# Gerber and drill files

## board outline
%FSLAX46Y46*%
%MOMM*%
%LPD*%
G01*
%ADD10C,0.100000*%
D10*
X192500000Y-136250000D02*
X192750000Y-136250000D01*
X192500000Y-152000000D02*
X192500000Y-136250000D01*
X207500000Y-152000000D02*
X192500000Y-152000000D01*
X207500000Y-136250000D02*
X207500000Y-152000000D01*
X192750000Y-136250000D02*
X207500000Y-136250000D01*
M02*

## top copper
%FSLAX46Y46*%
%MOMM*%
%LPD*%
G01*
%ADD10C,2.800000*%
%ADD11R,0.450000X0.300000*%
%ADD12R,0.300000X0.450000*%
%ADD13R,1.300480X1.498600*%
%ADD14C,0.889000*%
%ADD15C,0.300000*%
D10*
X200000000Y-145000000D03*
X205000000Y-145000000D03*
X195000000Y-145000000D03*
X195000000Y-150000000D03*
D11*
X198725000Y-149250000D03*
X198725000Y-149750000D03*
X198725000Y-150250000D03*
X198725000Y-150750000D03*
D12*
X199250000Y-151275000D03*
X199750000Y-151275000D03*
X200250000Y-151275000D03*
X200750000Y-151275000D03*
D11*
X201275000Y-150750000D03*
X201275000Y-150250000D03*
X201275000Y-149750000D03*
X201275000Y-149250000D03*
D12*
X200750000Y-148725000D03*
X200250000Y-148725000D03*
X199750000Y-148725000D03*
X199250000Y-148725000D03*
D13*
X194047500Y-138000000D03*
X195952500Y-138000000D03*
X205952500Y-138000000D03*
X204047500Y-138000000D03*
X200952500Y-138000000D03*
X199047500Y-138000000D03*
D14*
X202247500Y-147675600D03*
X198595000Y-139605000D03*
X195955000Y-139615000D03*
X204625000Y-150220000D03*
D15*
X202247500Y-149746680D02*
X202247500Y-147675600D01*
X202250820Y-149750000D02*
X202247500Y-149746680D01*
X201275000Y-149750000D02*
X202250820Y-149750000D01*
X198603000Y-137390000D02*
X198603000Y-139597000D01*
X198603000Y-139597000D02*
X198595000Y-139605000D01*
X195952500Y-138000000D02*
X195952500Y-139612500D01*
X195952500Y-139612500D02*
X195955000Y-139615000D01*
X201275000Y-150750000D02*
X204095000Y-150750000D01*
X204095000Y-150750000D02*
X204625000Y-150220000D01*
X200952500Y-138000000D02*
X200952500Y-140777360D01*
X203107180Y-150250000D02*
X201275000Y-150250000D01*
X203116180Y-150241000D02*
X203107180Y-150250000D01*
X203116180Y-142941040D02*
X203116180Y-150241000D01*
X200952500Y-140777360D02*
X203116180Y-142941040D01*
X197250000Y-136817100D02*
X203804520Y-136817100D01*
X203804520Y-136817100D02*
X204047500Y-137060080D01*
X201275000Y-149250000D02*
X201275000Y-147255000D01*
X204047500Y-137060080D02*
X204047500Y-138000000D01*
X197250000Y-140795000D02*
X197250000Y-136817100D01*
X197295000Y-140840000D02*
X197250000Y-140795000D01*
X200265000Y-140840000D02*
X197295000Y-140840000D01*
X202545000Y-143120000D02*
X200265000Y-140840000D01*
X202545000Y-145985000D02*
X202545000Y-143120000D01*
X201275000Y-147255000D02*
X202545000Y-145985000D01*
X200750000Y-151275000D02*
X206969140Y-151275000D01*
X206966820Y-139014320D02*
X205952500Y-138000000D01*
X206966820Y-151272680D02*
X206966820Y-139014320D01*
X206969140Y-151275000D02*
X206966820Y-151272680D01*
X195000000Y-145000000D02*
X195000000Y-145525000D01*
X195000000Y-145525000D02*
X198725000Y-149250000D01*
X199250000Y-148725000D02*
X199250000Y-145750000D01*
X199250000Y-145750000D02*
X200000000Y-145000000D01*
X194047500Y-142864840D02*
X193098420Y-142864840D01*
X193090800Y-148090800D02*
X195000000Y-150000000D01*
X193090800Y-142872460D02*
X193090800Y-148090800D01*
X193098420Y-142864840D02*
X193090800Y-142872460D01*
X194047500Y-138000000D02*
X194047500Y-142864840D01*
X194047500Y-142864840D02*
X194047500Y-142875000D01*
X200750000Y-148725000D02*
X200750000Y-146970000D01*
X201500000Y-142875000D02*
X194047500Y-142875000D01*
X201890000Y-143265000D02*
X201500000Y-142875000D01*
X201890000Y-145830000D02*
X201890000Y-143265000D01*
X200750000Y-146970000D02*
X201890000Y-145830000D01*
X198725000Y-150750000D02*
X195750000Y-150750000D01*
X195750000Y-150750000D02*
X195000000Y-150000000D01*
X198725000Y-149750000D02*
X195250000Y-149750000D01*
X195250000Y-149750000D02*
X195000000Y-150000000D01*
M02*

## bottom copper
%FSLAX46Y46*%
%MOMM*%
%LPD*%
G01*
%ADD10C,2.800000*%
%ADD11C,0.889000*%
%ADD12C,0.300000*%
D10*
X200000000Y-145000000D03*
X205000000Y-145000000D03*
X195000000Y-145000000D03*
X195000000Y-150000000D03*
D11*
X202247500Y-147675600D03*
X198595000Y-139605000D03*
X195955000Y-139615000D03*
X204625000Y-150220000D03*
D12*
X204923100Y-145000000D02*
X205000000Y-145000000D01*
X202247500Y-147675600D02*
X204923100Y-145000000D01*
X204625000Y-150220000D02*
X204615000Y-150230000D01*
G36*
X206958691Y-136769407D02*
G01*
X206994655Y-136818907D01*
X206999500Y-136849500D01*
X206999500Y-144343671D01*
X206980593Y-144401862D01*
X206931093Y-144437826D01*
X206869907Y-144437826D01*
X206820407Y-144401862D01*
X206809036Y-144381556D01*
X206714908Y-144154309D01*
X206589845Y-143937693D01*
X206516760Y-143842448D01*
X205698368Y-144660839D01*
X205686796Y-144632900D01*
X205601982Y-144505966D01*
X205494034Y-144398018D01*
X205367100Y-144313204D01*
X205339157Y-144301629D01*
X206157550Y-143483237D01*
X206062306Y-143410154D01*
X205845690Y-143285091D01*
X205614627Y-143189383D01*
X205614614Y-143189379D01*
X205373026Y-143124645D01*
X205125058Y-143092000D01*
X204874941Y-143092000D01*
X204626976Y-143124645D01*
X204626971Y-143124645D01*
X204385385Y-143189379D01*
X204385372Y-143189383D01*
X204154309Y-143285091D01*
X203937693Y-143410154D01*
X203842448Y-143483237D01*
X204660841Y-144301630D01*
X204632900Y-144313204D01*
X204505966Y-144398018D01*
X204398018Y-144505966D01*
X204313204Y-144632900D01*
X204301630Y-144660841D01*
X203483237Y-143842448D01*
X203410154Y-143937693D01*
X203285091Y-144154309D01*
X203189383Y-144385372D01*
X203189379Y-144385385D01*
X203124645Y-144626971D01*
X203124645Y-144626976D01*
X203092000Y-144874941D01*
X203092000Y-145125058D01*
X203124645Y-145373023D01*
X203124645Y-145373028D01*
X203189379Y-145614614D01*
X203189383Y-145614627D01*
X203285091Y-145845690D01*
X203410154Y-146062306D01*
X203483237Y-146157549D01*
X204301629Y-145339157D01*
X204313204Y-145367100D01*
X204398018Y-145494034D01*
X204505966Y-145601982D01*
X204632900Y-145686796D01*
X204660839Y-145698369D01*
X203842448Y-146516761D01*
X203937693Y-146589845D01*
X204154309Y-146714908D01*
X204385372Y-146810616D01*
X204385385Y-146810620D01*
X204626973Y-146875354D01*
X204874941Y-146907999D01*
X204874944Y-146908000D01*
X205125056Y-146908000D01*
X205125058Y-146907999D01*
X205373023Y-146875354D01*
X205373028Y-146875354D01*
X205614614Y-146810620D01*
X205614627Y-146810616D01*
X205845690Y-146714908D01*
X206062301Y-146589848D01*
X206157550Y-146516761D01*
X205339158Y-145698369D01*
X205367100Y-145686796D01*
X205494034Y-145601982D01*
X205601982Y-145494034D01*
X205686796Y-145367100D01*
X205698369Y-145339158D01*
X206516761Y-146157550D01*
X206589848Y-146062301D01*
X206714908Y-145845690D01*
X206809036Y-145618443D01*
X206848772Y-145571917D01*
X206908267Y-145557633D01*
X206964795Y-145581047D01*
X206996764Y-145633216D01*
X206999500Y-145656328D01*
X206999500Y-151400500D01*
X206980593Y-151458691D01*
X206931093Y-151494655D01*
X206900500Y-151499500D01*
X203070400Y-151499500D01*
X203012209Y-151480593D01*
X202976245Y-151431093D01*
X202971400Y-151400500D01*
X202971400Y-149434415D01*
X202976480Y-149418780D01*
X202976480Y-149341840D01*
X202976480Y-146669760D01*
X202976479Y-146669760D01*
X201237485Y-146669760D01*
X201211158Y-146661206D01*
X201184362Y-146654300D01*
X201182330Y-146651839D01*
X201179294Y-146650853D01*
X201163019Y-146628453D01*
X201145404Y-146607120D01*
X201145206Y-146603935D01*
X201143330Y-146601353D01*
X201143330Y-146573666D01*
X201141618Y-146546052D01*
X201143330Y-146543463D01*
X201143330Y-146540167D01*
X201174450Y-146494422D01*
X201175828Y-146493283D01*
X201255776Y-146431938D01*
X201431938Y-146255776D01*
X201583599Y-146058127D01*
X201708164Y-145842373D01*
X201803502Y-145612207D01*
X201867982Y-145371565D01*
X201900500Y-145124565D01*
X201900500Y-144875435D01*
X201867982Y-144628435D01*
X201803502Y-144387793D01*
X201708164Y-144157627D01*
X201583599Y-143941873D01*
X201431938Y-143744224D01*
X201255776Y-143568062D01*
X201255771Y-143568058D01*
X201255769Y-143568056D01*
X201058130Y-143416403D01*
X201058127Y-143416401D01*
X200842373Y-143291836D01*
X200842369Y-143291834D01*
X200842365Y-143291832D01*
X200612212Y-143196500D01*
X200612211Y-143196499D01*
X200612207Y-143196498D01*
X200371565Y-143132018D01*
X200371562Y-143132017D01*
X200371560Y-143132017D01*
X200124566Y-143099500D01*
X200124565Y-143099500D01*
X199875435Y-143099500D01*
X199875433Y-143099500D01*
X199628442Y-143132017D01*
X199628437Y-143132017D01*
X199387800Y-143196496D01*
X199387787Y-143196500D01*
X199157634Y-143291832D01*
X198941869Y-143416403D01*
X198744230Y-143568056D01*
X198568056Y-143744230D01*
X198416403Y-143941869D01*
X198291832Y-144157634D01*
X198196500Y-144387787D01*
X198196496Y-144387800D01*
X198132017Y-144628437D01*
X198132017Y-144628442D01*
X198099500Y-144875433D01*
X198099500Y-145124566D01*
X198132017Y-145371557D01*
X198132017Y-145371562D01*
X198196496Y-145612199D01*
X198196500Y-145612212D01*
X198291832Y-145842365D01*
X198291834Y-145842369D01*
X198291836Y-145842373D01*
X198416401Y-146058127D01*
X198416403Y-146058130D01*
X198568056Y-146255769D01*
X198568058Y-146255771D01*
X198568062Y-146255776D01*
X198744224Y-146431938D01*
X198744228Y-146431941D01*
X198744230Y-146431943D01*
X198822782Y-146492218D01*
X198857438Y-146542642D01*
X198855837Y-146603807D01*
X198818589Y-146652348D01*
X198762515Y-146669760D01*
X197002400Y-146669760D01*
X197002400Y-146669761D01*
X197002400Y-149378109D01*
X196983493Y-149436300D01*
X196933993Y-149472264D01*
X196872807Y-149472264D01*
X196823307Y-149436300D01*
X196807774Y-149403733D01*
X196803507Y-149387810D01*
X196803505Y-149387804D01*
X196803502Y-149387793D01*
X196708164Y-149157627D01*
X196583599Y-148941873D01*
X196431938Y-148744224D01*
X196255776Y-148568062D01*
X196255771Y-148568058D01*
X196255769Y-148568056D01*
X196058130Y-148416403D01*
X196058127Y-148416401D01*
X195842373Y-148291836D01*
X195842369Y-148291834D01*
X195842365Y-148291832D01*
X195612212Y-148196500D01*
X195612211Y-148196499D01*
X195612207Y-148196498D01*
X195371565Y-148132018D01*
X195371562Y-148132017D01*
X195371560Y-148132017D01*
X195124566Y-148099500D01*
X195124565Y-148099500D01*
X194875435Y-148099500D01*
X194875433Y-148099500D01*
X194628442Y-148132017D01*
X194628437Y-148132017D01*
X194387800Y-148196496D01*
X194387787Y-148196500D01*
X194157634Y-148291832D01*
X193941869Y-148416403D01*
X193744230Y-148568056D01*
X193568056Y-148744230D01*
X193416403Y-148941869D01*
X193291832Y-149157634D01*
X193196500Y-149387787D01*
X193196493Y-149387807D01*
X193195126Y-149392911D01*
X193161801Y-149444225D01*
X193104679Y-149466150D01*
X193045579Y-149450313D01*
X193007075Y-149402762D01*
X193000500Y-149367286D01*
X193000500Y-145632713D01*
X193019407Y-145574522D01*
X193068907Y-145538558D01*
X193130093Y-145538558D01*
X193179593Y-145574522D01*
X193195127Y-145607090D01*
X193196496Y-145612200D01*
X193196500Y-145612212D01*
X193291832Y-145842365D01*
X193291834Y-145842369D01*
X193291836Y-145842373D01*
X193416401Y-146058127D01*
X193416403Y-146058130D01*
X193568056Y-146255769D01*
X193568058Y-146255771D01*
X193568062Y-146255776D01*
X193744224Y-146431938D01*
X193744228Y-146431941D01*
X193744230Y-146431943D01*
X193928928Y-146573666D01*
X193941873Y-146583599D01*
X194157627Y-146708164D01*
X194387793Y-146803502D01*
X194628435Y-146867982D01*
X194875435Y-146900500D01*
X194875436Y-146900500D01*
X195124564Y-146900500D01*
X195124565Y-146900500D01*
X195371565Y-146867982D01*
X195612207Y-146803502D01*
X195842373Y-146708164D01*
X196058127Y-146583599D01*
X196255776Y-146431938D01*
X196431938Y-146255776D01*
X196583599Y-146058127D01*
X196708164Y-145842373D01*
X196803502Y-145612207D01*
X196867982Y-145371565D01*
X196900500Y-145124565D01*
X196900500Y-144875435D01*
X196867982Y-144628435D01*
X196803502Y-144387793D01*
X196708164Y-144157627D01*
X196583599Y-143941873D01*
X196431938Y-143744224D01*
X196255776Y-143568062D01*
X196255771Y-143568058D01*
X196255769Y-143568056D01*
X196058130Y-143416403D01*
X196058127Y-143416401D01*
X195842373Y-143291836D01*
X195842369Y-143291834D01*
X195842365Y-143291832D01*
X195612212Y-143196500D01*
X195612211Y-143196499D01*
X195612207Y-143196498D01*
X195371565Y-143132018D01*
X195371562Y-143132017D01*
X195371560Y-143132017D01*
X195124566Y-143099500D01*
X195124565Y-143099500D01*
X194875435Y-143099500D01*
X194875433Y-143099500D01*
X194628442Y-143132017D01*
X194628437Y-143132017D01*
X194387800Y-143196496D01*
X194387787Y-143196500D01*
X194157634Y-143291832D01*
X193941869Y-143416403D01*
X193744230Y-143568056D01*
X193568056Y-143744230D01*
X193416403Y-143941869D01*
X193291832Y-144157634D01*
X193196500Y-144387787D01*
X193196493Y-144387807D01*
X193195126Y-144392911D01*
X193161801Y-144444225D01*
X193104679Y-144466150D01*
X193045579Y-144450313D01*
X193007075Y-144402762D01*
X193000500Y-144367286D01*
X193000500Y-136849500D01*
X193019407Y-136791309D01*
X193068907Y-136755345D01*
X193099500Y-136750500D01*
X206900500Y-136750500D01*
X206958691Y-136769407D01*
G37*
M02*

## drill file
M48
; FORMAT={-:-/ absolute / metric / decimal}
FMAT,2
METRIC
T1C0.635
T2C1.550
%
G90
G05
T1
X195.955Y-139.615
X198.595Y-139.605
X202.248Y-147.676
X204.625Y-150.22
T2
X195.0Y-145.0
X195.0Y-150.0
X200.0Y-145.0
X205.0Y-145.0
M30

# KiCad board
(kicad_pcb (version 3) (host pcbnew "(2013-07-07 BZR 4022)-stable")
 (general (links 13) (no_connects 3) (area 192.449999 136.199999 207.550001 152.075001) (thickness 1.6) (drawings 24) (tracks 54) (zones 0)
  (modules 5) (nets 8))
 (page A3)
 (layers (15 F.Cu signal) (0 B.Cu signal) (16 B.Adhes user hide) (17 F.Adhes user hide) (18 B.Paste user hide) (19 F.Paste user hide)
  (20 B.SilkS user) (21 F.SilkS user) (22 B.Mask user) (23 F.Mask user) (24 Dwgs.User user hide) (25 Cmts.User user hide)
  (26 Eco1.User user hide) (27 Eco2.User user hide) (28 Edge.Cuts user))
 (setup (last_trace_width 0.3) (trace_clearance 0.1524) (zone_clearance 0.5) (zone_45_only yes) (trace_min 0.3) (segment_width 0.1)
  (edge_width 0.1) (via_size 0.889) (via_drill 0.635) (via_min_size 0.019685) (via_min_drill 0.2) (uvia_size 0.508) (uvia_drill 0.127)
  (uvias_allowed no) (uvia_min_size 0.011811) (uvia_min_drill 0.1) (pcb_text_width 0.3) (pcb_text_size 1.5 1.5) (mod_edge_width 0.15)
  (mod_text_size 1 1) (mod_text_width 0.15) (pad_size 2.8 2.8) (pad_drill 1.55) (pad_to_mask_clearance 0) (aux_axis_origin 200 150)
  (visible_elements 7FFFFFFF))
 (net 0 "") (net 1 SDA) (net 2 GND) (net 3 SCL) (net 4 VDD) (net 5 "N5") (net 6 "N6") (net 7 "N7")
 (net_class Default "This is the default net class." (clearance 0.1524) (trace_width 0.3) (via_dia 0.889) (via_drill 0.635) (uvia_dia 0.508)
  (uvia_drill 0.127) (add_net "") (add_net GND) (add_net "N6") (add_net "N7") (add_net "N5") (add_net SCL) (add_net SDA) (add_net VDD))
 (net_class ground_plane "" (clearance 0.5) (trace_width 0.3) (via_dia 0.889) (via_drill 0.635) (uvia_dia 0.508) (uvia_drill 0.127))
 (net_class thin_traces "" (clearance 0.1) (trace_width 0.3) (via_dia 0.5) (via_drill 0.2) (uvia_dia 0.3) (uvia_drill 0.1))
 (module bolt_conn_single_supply (layer F.Cu) (at 200 150)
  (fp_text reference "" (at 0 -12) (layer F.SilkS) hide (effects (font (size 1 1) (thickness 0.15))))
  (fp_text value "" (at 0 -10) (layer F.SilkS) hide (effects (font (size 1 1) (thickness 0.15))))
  (pad 4 thru_hole circle (at 0 -5) (size 2.8 2.8) (drill 1.55) (layers *.Cu F.SilkS F.Mask) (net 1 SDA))
  (pad 2 thru_hole circle (at 5 -5) (size 2.8 2.8) (drill 1.55) (layers *.Cu F.SilkS F.Mask) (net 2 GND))
  (pad 3 thru_hole circle (at -5 -5) (size 2.8 2.8) (drill 1.55) (layers *.Cu F.SilkS F.Mask) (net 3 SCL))
  (pad 1 thru_hole circle (at -5 0) (size 2.8 2.8) (drill 1.55) (layers *.Cu F.SilkS F.Mask) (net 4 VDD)))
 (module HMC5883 (layer F.Cu) (at 200 150)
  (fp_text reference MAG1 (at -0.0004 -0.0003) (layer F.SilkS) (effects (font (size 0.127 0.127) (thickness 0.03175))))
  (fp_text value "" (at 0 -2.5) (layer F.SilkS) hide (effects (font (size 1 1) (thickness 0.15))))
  (pad 1 smd rect (at -1.275 -0.75) (size 0.45 0.3) (layers F.Cu F.Paste F.Mask) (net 3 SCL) (clearance 0.05) (zone_connect 1))
  (pad 2 smd rect (at -1.275 -0.25) (size 0.45 0.3) (layers F.Cu F.Paste F.Mask) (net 4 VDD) (clearance 0.05))
  (pad 3 smd rect (at -1.275 0.25) (size 0.45 0.3) (layers F.Cu F.Paste F.Mask) (clearance 0.05))
  (pad 4 smd rect (at -1.275 0.75) (size 0.45 0.3) (layers F.Cu F.Paste F.Mask) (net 4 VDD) (clearance 0.05))
  (pad 5 smd rect (at -0.75 1.275 90) (size 0.45 0.3) (layers F.Cu F.Paste F.Mask) (clearance 0.05))
  (pad 6 smd rect (at -0.25 1.275 90) (size 0.45 0.3) (layers F.Cu F.Paste F.Mask) (clearance 0.05))
  (pad 7 smd rect (at 0.25 1.275 90) (size 0.45 0.3) (layers F.Cu F.Paste F.Mask) (clearance 0.05))
  (pad 8 smd rect (at 0.75 1.275 90) (size 0.45 0.3) (layers F.Cu F.Paste F.Mask) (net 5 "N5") (clearance 0.05))
  (pad 9 smd rect (at 1.275 0.75) (size 0.45 0.3) (layers F.Cu F.Paste F.Mask) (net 2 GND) (clearance 0.05))
  (pad 10 smd rect (at 1.275 0.25) (size 0.45 0.3) (layers F.Cu F.Paste F.Mask) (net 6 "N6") (clearance 0.05))
  (pad 11 smd rect (at 1.275 -0.25) (size 0.45 0.3) (layers F.Cu F.Paste F.Mask) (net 2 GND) (clearance 0.05))
  (pad 12 smd rect (at 1.275 -0.75) (size 0.45 0.3) (layers F.Cu F.Paste F.Mask) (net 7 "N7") (clearance 0.05))
  (pad 13 smd rect (at 0.75 -1.275 90) (size 0.45 0.3) (layers F.Cu F.Paste F.Mask) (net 4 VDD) (clearance 0.05))
  (pad 14 smd rect (at 0.25 -1.275 90) (size 0.45 0.3) (layers F.Cu F.Paste F.Mask) (clearance 0.05))
  (pad 15 smd rect (at -0.25 -1.275 90) (size 0.45 0.3) (layers F.Cu F.Paste F.Mask) (clearance 0.05))
  (pad 16 smd rect (at -0.75 -1.275 90) (size 0.45 0.3) (layers F.Cu F.Paste F.Mask) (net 1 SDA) (clearance 0.05)))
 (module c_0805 (layer F.Cu) (at 195 138 180)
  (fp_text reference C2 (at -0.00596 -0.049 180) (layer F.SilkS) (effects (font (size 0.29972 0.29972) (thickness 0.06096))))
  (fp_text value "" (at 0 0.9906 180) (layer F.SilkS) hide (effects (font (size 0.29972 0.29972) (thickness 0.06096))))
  (pad 1 smd rect (at 0.9525 0 180) (size 1.30048 1.4986) (layers F.Cu F.Paste F.Mask) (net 4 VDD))
  (pad 2 smd rect (at -0.9525 0 180) (size 1.30048 1.4986) (layers F.Cu F.Paste F.Mask) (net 2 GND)))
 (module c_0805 (layer F.Cu) (at 205 138)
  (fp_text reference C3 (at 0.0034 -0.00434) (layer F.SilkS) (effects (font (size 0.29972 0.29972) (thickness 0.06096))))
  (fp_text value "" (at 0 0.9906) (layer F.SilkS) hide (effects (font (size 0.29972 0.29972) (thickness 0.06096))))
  (pad 1 smd rect (at 0.9525 0) (size 1.30048 1.4986) (layers F.Cu F.Paste F.Mask) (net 5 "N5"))
  (pad 2 smd rect (at -0.9525 0) (size 1.30048 1.4986) (layers F.Cu F.Paste F.Mask) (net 7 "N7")))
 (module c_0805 (layer F.Cu) (at 200 138)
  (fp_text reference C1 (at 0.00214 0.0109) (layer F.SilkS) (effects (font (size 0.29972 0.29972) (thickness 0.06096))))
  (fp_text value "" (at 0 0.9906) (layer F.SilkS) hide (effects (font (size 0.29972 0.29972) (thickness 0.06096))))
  (pad 1 smd rect (at 0.9525 0) (size 1.30048 1.4986) (layers F.Cu F.Paste F.Mask) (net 6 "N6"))
  (pad 2 smd rect (at -0.9525 0) (size 1.30048 1.4986) (layers F.Cu F.Paste F.Mask) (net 2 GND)))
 (gr_line (start 192.5 136.25) (end 192.75 136.25) (angle 90) (layer Edge.Cuts) (width 0.1))
 (gr_line (start 192.5 152) (end 192.5 136.25) (angle 90) (layer Edge.Cuts) (width 0.1))
 (gr_line (start 207.5 152) (end 192.5 152) (angle 90) (layer Edge.Cuts) (width 0.1))
 (gr_line (start 207.5 136.25) (end 207.5 152) (angle 90) (layer Edge.Cuts) (width 0.1))
 (gr_line (start 192.75 136.25) (end 207.5 136.25) (angle 90) (layer Edge.Cuts) (width 0.1))
 (segment (start 204.9231 145) (end 205 145) (width 0.3) (layer B.Cu) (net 2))
 (segment (start 202.2475 147.6756) (end 204.9231 145) (width 0.3) (layer B.Cu) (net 2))
 (via (at 202.2475 147.6756) (size 0.889) (layers F.Cu B.Cu) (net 2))
 (segment (start 202.2475 149.74668) (end 202.2475 147.6756) (width 0.3) (layer F.Cu) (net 2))
 (segment (start 202.25082 149.75) (end 202.2475 149.74668) (width 0.3) (layer F.Cu) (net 2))
 (segment (start 201.275 149.75) (end 202.25082 149.75) (width 0.3) (layer F.Cu) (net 2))
 (segment (start 198.603 137.39) (end 198.603 139.597) (width 0.3) (layer F.Cu) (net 2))
 (via (at 198.595 139.605) (size 0.889) (layers F.Cu B.Cu) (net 2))
 (segment (start 198.603 139.597) (end 198.595 139.605) (width 0.3) (layer F.Cu) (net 2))
 (segment (start 195.9525 138) (end 195.9525 139.6125) (width 0.3) (layer F.Cu) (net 2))
 (via (at 195.955 139.615) (size 0.889) (layers F.Cu B.Cu) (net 2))
 (segment (start 195.9525 139.6125) (end 195.955 139.615) (width 0.3) (layer F.Cu) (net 2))
 (segment (start 201.275 150.75) (end 204.095 150.75) (width 0.3) (layer F.Cu) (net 2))
 (segment (start 204.625 150.22) (end 204.615 150.23) (width 0.3) (layer B.Cu) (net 2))
 (via (at 204.625 150.22) (size 0.889) (layers F.Cu B.Cu) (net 2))
 (segment (start 204.095 150.75) (end 204.625 150.22) (width 0.3) (layer F.Cu) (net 2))
 (segment (start 200.9525 138) (end 200.9525 140.77736) (width 0.3) (layer F.Cu) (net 6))
 (segment (start 203.10718 150.25) (end 201.275 150.25) (width 0.3) (layer F.Cu) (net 6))
 (segment (start 203.11618 150.241) (end 203.10718 150.25) (width 0.3) (layer F.Cu) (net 6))
 (segment (start 203.11618 142.94104) (end 203.11618 150.241) (width 0.3) (layer F.Cu) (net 6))
 (segment (start 200.9525 140.77736) (end 203.11618 142.94104) (width 0.3) (layer F.Cu) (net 6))
 (segment (start 197.25 136.8171) (end 203.80452 136.8171) (width 0.3) (layer F.Cu) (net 7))
 (segment (start 203.80452 136.8171) (end 204.0475 137.06008) (width 0.3) (layer F.Cu) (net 7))
 (segment (start 201.275 149.25) (end 201.275 147.255) (width 0.3) (layer F.Cu) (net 7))
 (segment (start 204.0475 137.06008) (end 204.0475 138) (width 0.3) (layer F.Cu) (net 7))
 (segment (start 197.25 140.795) (end 197.25 136.8171) (width 0.3) (layer F.Cu) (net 7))
 (segment (start 197.295 140.84) (end 197.25 140.795) (width 0.3) (layer F.Cu) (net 7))
 (segment (start 200.265 140.84) (end 197.295 140.84) (width 0.3) (layer F.Cu) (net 7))
 (segment (start 202.545 143.12) (end 200.265 140.84) (width 0.3) (layer F.Cu) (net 7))
 (segment (start 202.545 145.985) (end 202.545 143.12) (width 0.3) (layer F.Cu) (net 7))
 (segment (start 201.275 147.255) (end 202.545 145.985) (width 0.3) (layer F.Cu) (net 7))
 (segment (start 200.75 151.275) (end 206.96914 151.275) (width 0.3) (layer F.Cu) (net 5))
 (segment (start 206.96682 139.01432) (end 205.9525 138) (width 0.3) (layer F.Cu) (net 5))
 (segment (start 206.96682 151.27268) (end 206.96682 139.01432) (width 0.3) (layer F.Cu) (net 5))
 (segment (start 206.96914 151.275) (end 206.96682 151.27268) (width 0.3) (layer F.Cu) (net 5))
 (segment (start 195 145) (end 195 145.525) (width 0.3) (layer F.Cu) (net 3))
 (segment (start 195 145.525) (end 198.725 149.25) (width 0.3) (layer F.Cu) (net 3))
 (segment (start 199.25 148.725) (end 199.25 145.75) (width 0.3) (layer F.Cu) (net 1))
 (segment (start 199.25 145.75) (end 200 145) (width 0.3) (layer F.Cu) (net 1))
 (segment (start 194.0475 142.86484) (end 193.09842 142.86484) (width 0.3) (layer F.Cu) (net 4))
 (segment (start 193.0908 148.0908) (end 195 150) (width 0.3) (layer F.Cu) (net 4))
 (segment (start 193.0908 142.87246) (end 193.0908 148.0908) (width 0.3) (layer F.Cu) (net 4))
 (segment (start 193.09842 142.86484) (end 193.0908 142.87246) (width 0.3) (layer F.Cu) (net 4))
 (segment (start 194.0475 138) (end 194.0475 142.86484) (width 0.3) (layer F.Cu) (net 4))
 (segment (start 194.0475 142.86484) (end 194.0475 142.875) (width 0.3) (layer F.Cu) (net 4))
 (segment (start 200.75 148.725) (end 200.75 146.97) (width 0.3) (layer F.Cu) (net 4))
 (segment (start 201.5 142.875) (end 194.0475 142.875) (width 0.3) (layer F.Cu) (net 4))
 (segment (start 201.89 143.265) (end 201.5 142.875) (width 0.3) (layer F.Cu) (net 4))
 (segment (start 201.89 145.83) (end 201.89 143.265) (width 0.3) (layer F.Cu) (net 4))
 (segment (start 200.75 146.97) (end 201.89 145.83) (width 0.3) (layer F.Cu) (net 4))
 (segment (start 198.725 150.75) (end 195.75 150.75) (width 0.3) (layer F.Cu) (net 4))
 (segment (start 195.75 150.75) (end 195 150) (width 0.3) (layer F.Cu) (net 4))
 (segment (start 198.725 149.75) (end 195.25 149.75) (width 0.3) (layer F.Cu) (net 4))
 (segment (start 195.25 149.75) (end 195 150) (width 0.3) (layer F.Cu) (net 4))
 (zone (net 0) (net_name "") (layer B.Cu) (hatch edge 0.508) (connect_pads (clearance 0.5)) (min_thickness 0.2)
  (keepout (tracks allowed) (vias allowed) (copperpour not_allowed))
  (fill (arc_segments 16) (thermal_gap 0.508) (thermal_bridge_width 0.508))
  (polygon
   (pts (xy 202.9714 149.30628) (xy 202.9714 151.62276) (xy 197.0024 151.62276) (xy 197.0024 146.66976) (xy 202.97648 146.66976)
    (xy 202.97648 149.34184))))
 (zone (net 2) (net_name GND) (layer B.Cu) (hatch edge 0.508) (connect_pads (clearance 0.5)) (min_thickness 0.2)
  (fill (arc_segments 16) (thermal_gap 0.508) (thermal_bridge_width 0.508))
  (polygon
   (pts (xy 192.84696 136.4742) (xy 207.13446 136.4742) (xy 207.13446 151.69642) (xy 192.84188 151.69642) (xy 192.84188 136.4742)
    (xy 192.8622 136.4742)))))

